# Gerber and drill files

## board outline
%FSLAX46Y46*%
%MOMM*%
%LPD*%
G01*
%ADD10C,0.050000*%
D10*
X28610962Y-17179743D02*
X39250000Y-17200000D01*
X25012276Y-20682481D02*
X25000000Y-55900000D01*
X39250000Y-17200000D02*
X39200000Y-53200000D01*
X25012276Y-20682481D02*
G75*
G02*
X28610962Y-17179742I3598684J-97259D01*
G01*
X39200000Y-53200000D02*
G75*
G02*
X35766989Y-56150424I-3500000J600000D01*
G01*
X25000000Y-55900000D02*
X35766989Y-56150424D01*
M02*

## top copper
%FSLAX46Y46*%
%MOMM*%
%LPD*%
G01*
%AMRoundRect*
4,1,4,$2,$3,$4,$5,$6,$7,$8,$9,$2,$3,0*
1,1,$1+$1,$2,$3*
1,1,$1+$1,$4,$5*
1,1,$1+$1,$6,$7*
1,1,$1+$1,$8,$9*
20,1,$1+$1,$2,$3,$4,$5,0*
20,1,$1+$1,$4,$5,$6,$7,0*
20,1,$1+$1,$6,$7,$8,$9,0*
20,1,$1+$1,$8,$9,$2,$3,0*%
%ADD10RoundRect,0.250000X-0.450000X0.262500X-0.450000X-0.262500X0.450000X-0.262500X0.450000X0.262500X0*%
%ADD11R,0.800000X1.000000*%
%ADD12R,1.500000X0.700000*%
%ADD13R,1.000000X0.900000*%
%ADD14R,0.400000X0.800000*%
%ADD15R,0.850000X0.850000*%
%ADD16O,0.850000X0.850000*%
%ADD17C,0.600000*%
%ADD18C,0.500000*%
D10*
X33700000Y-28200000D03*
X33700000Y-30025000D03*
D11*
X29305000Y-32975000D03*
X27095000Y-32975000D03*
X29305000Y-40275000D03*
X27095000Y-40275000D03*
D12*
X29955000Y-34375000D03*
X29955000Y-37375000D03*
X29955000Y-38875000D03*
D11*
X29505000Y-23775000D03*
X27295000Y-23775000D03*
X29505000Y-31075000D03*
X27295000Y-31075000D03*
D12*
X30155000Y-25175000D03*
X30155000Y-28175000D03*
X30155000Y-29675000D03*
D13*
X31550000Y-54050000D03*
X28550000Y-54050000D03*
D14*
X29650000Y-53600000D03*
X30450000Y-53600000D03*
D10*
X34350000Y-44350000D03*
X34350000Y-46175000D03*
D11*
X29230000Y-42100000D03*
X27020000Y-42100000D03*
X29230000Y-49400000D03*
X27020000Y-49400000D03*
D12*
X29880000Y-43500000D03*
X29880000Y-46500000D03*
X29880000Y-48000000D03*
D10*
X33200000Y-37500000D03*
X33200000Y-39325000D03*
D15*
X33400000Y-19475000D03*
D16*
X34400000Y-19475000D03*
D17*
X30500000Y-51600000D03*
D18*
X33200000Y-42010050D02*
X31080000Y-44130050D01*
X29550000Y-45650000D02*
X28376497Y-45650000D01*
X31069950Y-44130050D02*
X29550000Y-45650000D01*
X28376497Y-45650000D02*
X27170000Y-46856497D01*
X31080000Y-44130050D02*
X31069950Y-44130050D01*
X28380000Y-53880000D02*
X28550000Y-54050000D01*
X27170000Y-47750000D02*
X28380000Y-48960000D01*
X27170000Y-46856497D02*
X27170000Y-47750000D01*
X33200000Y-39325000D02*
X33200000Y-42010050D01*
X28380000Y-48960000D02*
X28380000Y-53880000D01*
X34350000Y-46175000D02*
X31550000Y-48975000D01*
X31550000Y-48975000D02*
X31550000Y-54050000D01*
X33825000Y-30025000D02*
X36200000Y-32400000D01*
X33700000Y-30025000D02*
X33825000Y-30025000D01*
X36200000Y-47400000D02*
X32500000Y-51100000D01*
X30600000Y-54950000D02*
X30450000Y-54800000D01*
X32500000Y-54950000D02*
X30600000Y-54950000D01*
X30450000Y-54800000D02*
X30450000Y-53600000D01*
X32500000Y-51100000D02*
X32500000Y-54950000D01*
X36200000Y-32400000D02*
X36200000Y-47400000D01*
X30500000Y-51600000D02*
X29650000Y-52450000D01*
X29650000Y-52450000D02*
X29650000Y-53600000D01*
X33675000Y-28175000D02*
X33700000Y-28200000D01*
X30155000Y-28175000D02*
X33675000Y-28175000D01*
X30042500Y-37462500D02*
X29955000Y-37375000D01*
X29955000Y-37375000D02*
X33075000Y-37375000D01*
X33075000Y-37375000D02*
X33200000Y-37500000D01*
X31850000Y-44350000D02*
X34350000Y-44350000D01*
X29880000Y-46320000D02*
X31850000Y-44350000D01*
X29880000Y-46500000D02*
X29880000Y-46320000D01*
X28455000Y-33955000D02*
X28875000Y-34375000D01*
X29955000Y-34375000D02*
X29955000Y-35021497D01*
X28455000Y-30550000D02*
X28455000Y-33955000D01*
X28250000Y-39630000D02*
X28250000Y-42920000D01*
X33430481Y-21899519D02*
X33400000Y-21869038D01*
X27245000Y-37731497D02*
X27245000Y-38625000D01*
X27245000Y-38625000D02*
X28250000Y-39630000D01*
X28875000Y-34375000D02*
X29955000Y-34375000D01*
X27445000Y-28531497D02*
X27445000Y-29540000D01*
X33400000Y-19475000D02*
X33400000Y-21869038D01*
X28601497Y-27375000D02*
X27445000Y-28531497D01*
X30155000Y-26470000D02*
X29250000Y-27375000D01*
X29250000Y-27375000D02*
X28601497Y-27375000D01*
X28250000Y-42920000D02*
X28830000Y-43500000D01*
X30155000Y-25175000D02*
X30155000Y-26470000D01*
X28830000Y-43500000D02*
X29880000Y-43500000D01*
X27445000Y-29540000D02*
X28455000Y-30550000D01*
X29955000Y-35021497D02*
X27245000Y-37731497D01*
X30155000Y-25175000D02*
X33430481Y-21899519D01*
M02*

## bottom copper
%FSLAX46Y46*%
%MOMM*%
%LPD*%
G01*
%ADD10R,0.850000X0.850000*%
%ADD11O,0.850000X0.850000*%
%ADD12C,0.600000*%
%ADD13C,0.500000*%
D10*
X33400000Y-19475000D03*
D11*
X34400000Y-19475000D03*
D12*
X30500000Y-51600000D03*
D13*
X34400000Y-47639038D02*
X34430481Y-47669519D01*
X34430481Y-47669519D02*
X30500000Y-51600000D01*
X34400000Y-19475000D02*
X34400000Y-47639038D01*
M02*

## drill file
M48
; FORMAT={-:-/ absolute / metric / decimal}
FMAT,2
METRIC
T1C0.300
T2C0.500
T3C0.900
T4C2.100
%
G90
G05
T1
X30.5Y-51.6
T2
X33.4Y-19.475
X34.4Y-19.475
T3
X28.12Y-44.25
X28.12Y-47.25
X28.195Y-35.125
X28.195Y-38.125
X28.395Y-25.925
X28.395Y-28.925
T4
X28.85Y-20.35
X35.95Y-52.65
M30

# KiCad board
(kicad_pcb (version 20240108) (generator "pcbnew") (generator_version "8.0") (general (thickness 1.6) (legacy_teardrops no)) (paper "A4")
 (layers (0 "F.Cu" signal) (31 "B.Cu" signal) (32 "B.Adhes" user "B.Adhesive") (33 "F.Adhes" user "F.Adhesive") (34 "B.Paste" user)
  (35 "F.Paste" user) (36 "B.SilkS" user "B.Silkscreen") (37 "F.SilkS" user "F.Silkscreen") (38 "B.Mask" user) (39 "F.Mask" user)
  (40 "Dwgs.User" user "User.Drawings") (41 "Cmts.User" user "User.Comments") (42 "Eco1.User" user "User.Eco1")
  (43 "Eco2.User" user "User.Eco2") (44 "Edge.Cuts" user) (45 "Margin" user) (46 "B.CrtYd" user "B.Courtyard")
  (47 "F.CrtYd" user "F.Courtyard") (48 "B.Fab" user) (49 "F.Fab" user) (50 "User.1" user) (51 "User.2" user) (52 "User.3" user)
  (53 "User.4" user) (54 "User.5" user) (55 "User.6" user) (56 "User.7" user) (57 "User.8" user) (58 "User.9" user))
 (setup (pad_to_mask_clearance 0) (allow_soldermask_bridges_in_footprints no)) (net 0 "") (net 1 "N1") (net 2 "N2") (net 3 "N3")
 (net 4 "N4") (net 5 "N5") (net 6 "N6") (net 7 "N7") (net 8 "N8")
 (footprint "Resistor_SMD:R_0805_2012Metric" (layer "F.Cu") (at 33.7 29.1125 -90)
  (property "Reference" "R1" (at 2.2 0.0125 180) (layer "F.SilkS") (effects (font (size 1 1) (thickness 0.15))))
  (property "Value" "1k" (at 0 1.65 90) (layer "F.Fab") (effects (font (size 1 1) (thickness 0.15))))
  (pad "1" smd roundrect (at -0.9125 0 270) (size 1.025 1.4) (layers "F.Cu" "F.Paste" "F.Mask") (roundrect_rratio 0.243902) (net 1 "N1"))
  (pad "2" smd roundrect (at 0.9125 0 270) (size 1.025 1.4) (layers "F.Cu" "F.Paste" "F.Mask") (roundrect_rratio 0.243902) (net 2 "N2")))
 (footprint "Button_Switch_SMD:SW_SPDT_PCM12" (layer "F.Cu") (at 28.525 36.625 -90)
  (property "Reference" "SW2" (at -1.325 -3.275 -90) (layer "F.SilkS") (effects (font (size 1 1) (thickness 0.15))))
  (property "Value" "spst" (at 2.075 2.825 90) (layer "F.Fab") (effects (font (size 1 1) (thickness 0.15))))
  (pad "" smd rect (at -3.65 -0.78 270) (size 1 0.8) (layers "F.Cu" "F.Paste" "F.Mask"))
  (pad "" smd rect (at -3.65 1.43 270) (size 1 0.8) (layers "F.Cu" "F.Paste" "F.Mask"))
  (pad "" np_thru_hole circle (at -1.5 0.33 270) (size 0.9 0.9) (drill 0.9) (layers "*.Cu" "*.Mask"))
  (pad "" np_thru_hole circle (at 1.5 0.33 270) (size 0.9 0.9) (drill 0.9) (layers "*.Cu" "*.Mask"))
  (pad "" smd rect (at 3.65 -0.78 270) (size 1 0.8) (layers "F.Cu" "F.Paste" "F.Mask"))
  (pad "" smd rect (at 3.65 1.43 270) (size 1 0.8) (layers "F.Cu" "F.Paste" "F.Mask"))
  (pad "1" smd rect (at -2.25 -1.43 270) (size 0.7 1.5) (layers "F.Cu" "F.Paste" "F.Mask") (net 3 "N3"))
  (pad "2" smd rect (at 0.75 -1.43 270) (size 0.7 1.5) (layers "F.Cu" "F.Paste" "F.Mask") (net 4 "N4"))
  (pad "3" smd rect (at 2.25 -1.43 270) (size 0.7 1.5) (layers "F.Cu" "F.Paste" "F.Mask")))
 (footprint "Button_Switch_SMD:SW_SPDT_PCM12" (layer "F.Cu") (at 28.725 27.425 -90)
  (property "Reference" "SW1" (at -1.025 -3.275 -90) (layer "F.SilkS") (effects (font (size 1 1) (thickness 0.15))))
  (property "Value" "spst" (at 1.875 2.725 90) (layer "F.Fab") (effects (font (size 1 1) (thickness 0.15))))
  (pad "" smd rect (at -3.65 -0.78 270) (size 1 0.8) (layers "F.Cu" "F.Paste" "F.Mask"))
  (pad "" smd rect (at -3.65 1.43 270) (size 1 0.8) (layers "F.Cu" "F.Paste" "F.Mask"))
  (pad "" np_thru_hole circle (at -1.5 0.33 270) (size 0.9 0.9) (drill 0.9) (layers "*.Cu" "*.Mask"))
  (pad "" np_thru_hole circle (at 1.5 0.33 270) (size 0.9 0.9) (drill 0.9) (layers "*.Cu" "*.Mask"))
  (pad "" smd rect (at 3.65 -0.78 270) (size 1 0.8) (layers "F.Cu" "F.Paste" "F.Mask"))
  (pad "" smd rect (at 3.65 1.43 270) (size 1 0.8) (layers "F.Cu" "F.Paste" "F.Mask"))
  (pad "1" smd rect (at -2.25 -1.43 270) (size 0.7 1.5) (layers "F.Cu" "F.Paste" "F.Mask") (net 3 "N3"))
  (pad "2" smd rect (at 0.75 -1.43 270) (size 0.7 1.5) (layers "F.Cu" "F.Paste" "F.Mask") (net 1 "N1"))
  (pad "3" smd rect (at 2.25 -1.43 270) (size 0.7 1.5) (layers "F.Cu" "F.Paste" "F.Mask")))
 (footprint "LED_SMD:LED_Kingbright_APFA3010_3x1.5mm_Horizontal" (layer "F.Cu") (at 30.05 54.05 180)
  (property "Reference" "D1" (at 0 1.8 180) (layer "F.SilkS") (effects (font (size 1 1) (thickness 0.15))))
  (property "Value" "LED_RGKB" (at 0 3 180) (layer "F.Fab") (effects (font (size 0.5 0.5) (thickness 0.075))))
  (pad "1" smd rect (at -1.5 0 180) (size 1 0.9) (layers "F.Cu" "F.Paste" "F.Mask") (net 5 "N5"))
  (pad "2" smd rect (at 1.5 0 180) (size 1 0.9) (layers "F.Cu" "F.Paste" "F.Mask") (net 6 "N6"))
  (pad "3" smd rect (at 0.4 0.45 180) (size 0.4 0.8) (layers "F.Cu" "F.Paste" "F.Mask") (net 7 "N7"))
  (pad "4" smd rect (at -0.4 0.45 180) (size 0.4 0.8) (layers "F.Cu" "F.Paste" "F.Mask") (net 2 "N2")))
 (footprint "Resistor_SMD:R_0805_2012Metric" (layer "F.Cu") (at 34.35 45.2625 -90)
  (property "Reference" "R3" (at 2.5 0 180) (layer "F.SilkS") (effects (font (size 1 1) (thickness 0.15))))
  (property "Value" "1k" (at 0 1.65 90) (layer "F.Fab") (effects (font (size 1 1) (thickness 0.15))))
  (pad "1" smd roundrect (at -0.9125 0 270) (size 1.025 1.4) (layers "F.Cu" "F.Paste" "F.Mask") (roundrect_rratio 0.243902) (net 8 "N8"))
  (pad "2" smd roundrect (at 0.9125 0 270) (size 1.025 1.4) (layers "F.Cu" "F.Paste" "F.Mask") (roundrect_rratio 0.243902) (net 5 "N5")))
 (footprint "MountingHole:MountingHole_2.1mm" (layer "F.Cu") (at 35.95 52.65)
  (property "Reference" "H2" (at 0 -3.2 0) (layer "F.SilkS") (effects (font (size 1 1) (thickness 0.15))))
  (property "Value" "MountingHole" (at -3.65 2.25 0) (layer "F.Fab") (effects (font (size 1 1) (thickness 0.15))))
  (pad "" np_thru_hole circle (at 0 0) (size 2.1 2.1) (drill 2.1) (layers "*.Cu" "*.Mask")))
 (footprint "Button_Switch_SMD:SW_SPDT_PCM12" (layer "F.Cu") (at 28.45 45.75 -90)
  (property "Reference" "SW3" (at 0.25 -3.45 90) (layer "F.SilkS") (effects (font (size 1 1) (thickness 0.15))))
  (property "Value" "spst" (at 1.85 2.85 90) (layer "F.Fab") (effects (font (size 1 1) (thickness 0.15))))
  (pad "" smd rect (at -3.65 -0.78 270) (size 1 0.8) (layers "F.Cu" "F.Paste" "F.Mask"))
  (pad "" smd rect (at -3.65 1.43 270) (size 1 0.8) (layers "F.Cu" "F.Paste" "F.Mask"))
  (pad "" np_thru_hole circle (at -1.5 0.33 270) (size 0.9 0.9) (drill 0.9) (layers "*.Cu" "*.Mask"))
  (pad "" np_thru_hole circle (at 1.5 0.33 270) (size 0.9 0.9) (drill 0.9) (layers "*.Cu" "*.Mask"))
  (pad "" smd rect (at 3.65 -0.78 270) (size 1 0.8) (layers "F.Cu" "F.Paste" "F.Mask"))
  (pad "" smd rect (at 3.65 1.43 270) (size 1 0.8) (layers "F.Cu" "F.Paste" "F.Mask"))
  (pad "1" smd rect (at -2.25 -1.43 270) (size 0.7 1.5) (layers "F.Cu" "F.Paste" "F.Mask") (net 3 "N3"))
  (pad "2" smd rect (at 0.75 -1.43 270) (size 0.7 1.5) (layers "F.Cu" "F.Paste" "F.Mask") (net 8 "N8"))
  (pad "3" smd rect (at 2.25 -1.43 270) (size 0.7 1.5) (layers "F.Cu" "F.Paste" "F.Mask")))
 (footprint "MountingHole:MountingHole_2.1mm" (layer "F.Cu") (at 28.85 20.35)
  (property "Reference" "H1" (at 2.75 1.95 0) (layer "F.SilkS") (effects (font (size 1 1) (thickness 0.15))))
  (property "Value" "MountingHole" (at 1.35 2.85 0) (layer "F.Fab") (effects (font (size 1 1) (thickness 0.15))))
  (pad "" np_thru_hole circle (at 0 0) (size 2.1 2.1) (drill 2.1) (layers "*.Cu" "*.Mask")))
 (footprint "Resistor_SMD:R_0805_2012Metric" (layer "F.Cu") (at 33.2 38.4125 -90)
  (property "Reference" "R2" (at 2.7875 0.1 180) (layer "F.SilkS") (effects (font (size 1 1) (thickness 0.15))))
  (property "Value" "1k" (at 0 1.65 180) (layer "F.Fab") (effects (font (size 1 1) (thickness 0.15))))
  (pad "1" smd roundrect (at -0.9125 0 270) (size 1.025 1.4) (layers "F.Cu" "F.Paste" "F.Mask") (roundrect_rratio 0.243902) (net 4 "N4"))
  (pad "2" smd roundrect (at 0.9125 0 270) (size 1.025 1.4) (layers "F.Cu" "F.Paste" "F.Mask") (roundrect_rratio 0.243902) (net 6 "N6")))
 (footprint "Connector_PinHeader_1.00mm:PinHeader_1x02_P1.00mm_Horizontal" (layer "F.Cu") (at 33.4 19.475 90)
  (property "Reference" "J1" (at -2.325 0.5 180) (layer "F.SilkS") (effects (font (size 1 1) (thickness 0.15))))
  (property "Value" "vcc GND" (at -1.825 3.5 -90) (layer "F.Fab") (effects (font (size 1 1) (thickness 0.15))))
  (pad "1" thru_hole rect (at 0 0 90) (size 0.85 0.85) (drill 0.5) (layers "*.Cu" "*.Mask") (remove_unused_layers no) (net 3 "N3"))
  (pad "2" thru_hole oval (at 0 1 90) (size 0.85 0.85) (drill 0.5) (layers "*.Cu" "*.Mask") (remove_unused_layers no) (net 7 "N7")))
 (gr_line (start 28.610962 17.179743) (end 39.25 17.2) (stroke (width 0.05) (type default)) (layer "Edge.Cuts"))
 (gr_line (start 25.012276 20.682481) (end 25 55.9) (stroke (width 0.05) (type default)) (layer "Edge.Cuts"))
 (gr_line (start 39.25 17.2) (end 39.2 53.2) (stroke (width 0.05) (type default)) (layer "Edge.Cuts"))
 (gr_arc (start 25.012276 20.682481) (mid 26.1 18.2) (end 28.610962 17.179743) (stroke (width 0.05) (type default)) (layer "Edge.Cuts"))
 (gr_arc (start 39.2 53.2) (mid 38.014542 55.29312) (end 35.766989 56.150424) (stroke (width 0.05) (type default)) (layer "Edge.Cuts"))
 (gr_line (start 25 55.9) (end 35.766989 56.150424) (stroke (width 0.05) (type default)) (layer "Edge.Cuts"))
 (segment (start 33.2 42.01005) (end 31.08 44.13005) (width 0.5) (layer "F.Cu") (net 6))
 (segment (start 29.55 45.65) (end 28.376497 45.65) (width 0.5) (layer "F.Cu") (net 6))
 (segment (start 31.06995 44.13005) (end 29.55 45.65) (width 0.5) (layer "F.Cu") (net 6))
 (segment (start 28.376497 45.65) (end 27.17 46.856497) (width 0.5) (layer "F.Cu") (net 6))
 (segment (start 31.08 44.13005) (end 31.06995 44.13005) (width 0.5) (layer "F.Cu") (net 6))
 (segment (start 28.38 53.88) (end 28.55 54.05) (width 0.5) (layer "F.Cu") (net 6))
 (segment (start 27.17 47.75) (end 28.38 48.96) (width 0.5) (layer "F.Cu") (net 6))
 (segment (start 27.17 46.856497) (end 27.17 47.75) (width 0.5) (layer "F.Cu") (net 6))
 (segment (start 33.2 39.325) (end 33.2 42.01005) (width 0.5) (layer "F.Cu") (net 6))
 (segment (start 28.38 48.96) (end 28.38 53.88) (width 0.5) (layer "F.Cu") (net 6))
 (segment (start 34.35 46.175) (end 31.55 48.975) (width 0.5) (layer "F.Cu") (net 5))
 (segment (start 31.55 48.975) (end 31.55 54.05) (width 0.5) (layer "F.Cu") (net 5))
 (segment (start 33.825 30.025) (end 36.2 32.4) (width 0.5) (layer "F.Cu") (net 2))
 (segment (start 33.7 30.025) (end 33.825 30.025) (width 0.5) (layer "F.Cu") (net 2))
 (segment (start 36.2 47.4) (end 32.5 51.1) (width 0.5) (layer "F.Cu") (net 2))
 (segment (start 30.6 54.95) (end 30.45 54.8) (width 0.5) (layer "F.Cu") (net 2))
 (segment (start 32.5 54.95) (end 30.6 54.95) (width 0.5) (layer "F.Cu") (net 2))
 (segment (start 30.45 54.8) (end 30.45 53.6) (width 0.5) (layer "F.Cu") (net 2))
 (segment (start 32.5 51.1) (end 32.5 54.95) (width 0.5) (layer "F.Cu") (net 2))
 (segment (start 36.2 32.4) (end 36.2 47.4) (width 0.5) (layer "F.Cu") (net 2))
 (segment (start 30.5 51.6) (end 29.65 52.45) (width 0.5) (layer "F.Cu") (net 7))
 (segment (start 29.65 52.45) (end 29.65 53.6) (width 0.5) (layer "F.Cu") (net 7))
 (via (at 30.5 51.6) (size 0.6) (drill 0.3) (layers "F.Cu" "B.Cu") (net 7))
 (segment (start 34.4 47.639038) (end 34.430481 47.669519) (width 0.5) (layer "B.Cu") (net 7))
 (segment (start 34.430481 47.669519) (end 30.5 51.6) (width 0.5) (layer "B.Cu") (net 7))
 (segment (start 34.4 19.475) (end 34.4 47.639038) (width 0.5) (layer "B.Cu") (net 7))
 (segment (start 33.675 28.175) (end 33.7 28.2) (width 0.5) (layer "F.Cu") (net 1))
 (segment (start 30.155 28.175) (end 33.675 28.175) (width 0.5) (layer "F.Cu") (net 1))
 (segment (start 30.0425 37.4625) (end 29.955 37.375) (width 0.5) (layer "F.Cu") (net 4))
 (segment (start 29.955 37.375) (end 33.075 37.375) (width 0.5) (layer "F.Cu") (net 4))
 (segment (start 33.075 37.375) (end 33.2 37.5) (width 0.5) (layer "F.Cu") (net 4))
 (segment (start 31.85 44.35) (end 34.35 44.35) (width 0.5) (layer "F.Cu") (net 8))
 (segment (start 29.88 46.32) (end 31.85 44.35) (width 0.5) (layer "F.Cu") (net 8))
 (segment (start 29.88 46.5) (end 29.88 46.32) (width 0.5) (layer "F.Cu") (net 8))
 (segment (start 28.455 33.955) (end 28.875 34.375) (width 0.5) (layer "F.Cu") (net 3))
 (segment (start 29.955 34.375) (end 29.955 35.021497) (width 0.5) (layer "F.Cu") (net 3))
 (segment (start 28.455 30.55) (end 28.455 33.955) (width 0.5) (layer "F.Cu") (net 3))
 (segment (start 28.25 39.63) (end 28.25 42.92) (width 0.5) (layer "F.Cu") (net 3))
 (segment (start 33.430481 21.899519) (end 33.4 21.869038) (width 0.5) (layer "F.Cu") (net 3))
 (segment (start 27.245 37.731497) (end 27.245 38.625) (width 0.5) (layer "F.Cu") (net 3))
 (segment (start 27.245 38.625) (end 28.25 39.63) (width 0.5) (layer "F.Cu") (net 3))
 (segment (start 28.875 34.375) (end 29.955 34.375) (width 0.5) (layer "F.Cu") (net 3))
 (segment (start 27.445 28.531497) (end 27.445 29.54) (width 0.5) (layer "F.Cu") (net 3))
 (segment (start 33.4 19.475) (end 33.4 21.869038) (width 0.5) (layer "F.Cu") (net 3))
 (segment (start 28.601497 27.375) (end 27.445 28.531497) (width 0.5) (layer "F.Cu") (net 3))
 (segment (start 30.155 26.47) (end 29.25 27.375) (width 0.5) (layer "F.Cu") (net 3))
 (segment (start 29.25 27.375) (end 28.601497 27.375) (width 0.5) (layer "F.Cu") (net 3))
 (segment (start 28.25 42.92) (end 28.83 43.5) (width 0.5) (layer "F.Cu") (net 3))
 (segment (start 30.155 25.175) (end 30.155 26.47) (width 0.5) (layer "F.Cu") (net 3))
 (segment (start 28.83 43.5) (end 29.88 43.5) (width 0.5) (layer "F.Cu") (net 3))
 (segment (start 27.445 29.54) (end 28.455 30.55) (width 0.5) (layer "F.Cu") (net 3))
 (segment (start 29.955 35.021497) (end 27.245 37.731497) (width 0.5) (layer "F.Cu") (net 3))
 (segment (start 30.155 25.175) (end 33.430481 21.899519) (width 0.5) (layer "F.Cu") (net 3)))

